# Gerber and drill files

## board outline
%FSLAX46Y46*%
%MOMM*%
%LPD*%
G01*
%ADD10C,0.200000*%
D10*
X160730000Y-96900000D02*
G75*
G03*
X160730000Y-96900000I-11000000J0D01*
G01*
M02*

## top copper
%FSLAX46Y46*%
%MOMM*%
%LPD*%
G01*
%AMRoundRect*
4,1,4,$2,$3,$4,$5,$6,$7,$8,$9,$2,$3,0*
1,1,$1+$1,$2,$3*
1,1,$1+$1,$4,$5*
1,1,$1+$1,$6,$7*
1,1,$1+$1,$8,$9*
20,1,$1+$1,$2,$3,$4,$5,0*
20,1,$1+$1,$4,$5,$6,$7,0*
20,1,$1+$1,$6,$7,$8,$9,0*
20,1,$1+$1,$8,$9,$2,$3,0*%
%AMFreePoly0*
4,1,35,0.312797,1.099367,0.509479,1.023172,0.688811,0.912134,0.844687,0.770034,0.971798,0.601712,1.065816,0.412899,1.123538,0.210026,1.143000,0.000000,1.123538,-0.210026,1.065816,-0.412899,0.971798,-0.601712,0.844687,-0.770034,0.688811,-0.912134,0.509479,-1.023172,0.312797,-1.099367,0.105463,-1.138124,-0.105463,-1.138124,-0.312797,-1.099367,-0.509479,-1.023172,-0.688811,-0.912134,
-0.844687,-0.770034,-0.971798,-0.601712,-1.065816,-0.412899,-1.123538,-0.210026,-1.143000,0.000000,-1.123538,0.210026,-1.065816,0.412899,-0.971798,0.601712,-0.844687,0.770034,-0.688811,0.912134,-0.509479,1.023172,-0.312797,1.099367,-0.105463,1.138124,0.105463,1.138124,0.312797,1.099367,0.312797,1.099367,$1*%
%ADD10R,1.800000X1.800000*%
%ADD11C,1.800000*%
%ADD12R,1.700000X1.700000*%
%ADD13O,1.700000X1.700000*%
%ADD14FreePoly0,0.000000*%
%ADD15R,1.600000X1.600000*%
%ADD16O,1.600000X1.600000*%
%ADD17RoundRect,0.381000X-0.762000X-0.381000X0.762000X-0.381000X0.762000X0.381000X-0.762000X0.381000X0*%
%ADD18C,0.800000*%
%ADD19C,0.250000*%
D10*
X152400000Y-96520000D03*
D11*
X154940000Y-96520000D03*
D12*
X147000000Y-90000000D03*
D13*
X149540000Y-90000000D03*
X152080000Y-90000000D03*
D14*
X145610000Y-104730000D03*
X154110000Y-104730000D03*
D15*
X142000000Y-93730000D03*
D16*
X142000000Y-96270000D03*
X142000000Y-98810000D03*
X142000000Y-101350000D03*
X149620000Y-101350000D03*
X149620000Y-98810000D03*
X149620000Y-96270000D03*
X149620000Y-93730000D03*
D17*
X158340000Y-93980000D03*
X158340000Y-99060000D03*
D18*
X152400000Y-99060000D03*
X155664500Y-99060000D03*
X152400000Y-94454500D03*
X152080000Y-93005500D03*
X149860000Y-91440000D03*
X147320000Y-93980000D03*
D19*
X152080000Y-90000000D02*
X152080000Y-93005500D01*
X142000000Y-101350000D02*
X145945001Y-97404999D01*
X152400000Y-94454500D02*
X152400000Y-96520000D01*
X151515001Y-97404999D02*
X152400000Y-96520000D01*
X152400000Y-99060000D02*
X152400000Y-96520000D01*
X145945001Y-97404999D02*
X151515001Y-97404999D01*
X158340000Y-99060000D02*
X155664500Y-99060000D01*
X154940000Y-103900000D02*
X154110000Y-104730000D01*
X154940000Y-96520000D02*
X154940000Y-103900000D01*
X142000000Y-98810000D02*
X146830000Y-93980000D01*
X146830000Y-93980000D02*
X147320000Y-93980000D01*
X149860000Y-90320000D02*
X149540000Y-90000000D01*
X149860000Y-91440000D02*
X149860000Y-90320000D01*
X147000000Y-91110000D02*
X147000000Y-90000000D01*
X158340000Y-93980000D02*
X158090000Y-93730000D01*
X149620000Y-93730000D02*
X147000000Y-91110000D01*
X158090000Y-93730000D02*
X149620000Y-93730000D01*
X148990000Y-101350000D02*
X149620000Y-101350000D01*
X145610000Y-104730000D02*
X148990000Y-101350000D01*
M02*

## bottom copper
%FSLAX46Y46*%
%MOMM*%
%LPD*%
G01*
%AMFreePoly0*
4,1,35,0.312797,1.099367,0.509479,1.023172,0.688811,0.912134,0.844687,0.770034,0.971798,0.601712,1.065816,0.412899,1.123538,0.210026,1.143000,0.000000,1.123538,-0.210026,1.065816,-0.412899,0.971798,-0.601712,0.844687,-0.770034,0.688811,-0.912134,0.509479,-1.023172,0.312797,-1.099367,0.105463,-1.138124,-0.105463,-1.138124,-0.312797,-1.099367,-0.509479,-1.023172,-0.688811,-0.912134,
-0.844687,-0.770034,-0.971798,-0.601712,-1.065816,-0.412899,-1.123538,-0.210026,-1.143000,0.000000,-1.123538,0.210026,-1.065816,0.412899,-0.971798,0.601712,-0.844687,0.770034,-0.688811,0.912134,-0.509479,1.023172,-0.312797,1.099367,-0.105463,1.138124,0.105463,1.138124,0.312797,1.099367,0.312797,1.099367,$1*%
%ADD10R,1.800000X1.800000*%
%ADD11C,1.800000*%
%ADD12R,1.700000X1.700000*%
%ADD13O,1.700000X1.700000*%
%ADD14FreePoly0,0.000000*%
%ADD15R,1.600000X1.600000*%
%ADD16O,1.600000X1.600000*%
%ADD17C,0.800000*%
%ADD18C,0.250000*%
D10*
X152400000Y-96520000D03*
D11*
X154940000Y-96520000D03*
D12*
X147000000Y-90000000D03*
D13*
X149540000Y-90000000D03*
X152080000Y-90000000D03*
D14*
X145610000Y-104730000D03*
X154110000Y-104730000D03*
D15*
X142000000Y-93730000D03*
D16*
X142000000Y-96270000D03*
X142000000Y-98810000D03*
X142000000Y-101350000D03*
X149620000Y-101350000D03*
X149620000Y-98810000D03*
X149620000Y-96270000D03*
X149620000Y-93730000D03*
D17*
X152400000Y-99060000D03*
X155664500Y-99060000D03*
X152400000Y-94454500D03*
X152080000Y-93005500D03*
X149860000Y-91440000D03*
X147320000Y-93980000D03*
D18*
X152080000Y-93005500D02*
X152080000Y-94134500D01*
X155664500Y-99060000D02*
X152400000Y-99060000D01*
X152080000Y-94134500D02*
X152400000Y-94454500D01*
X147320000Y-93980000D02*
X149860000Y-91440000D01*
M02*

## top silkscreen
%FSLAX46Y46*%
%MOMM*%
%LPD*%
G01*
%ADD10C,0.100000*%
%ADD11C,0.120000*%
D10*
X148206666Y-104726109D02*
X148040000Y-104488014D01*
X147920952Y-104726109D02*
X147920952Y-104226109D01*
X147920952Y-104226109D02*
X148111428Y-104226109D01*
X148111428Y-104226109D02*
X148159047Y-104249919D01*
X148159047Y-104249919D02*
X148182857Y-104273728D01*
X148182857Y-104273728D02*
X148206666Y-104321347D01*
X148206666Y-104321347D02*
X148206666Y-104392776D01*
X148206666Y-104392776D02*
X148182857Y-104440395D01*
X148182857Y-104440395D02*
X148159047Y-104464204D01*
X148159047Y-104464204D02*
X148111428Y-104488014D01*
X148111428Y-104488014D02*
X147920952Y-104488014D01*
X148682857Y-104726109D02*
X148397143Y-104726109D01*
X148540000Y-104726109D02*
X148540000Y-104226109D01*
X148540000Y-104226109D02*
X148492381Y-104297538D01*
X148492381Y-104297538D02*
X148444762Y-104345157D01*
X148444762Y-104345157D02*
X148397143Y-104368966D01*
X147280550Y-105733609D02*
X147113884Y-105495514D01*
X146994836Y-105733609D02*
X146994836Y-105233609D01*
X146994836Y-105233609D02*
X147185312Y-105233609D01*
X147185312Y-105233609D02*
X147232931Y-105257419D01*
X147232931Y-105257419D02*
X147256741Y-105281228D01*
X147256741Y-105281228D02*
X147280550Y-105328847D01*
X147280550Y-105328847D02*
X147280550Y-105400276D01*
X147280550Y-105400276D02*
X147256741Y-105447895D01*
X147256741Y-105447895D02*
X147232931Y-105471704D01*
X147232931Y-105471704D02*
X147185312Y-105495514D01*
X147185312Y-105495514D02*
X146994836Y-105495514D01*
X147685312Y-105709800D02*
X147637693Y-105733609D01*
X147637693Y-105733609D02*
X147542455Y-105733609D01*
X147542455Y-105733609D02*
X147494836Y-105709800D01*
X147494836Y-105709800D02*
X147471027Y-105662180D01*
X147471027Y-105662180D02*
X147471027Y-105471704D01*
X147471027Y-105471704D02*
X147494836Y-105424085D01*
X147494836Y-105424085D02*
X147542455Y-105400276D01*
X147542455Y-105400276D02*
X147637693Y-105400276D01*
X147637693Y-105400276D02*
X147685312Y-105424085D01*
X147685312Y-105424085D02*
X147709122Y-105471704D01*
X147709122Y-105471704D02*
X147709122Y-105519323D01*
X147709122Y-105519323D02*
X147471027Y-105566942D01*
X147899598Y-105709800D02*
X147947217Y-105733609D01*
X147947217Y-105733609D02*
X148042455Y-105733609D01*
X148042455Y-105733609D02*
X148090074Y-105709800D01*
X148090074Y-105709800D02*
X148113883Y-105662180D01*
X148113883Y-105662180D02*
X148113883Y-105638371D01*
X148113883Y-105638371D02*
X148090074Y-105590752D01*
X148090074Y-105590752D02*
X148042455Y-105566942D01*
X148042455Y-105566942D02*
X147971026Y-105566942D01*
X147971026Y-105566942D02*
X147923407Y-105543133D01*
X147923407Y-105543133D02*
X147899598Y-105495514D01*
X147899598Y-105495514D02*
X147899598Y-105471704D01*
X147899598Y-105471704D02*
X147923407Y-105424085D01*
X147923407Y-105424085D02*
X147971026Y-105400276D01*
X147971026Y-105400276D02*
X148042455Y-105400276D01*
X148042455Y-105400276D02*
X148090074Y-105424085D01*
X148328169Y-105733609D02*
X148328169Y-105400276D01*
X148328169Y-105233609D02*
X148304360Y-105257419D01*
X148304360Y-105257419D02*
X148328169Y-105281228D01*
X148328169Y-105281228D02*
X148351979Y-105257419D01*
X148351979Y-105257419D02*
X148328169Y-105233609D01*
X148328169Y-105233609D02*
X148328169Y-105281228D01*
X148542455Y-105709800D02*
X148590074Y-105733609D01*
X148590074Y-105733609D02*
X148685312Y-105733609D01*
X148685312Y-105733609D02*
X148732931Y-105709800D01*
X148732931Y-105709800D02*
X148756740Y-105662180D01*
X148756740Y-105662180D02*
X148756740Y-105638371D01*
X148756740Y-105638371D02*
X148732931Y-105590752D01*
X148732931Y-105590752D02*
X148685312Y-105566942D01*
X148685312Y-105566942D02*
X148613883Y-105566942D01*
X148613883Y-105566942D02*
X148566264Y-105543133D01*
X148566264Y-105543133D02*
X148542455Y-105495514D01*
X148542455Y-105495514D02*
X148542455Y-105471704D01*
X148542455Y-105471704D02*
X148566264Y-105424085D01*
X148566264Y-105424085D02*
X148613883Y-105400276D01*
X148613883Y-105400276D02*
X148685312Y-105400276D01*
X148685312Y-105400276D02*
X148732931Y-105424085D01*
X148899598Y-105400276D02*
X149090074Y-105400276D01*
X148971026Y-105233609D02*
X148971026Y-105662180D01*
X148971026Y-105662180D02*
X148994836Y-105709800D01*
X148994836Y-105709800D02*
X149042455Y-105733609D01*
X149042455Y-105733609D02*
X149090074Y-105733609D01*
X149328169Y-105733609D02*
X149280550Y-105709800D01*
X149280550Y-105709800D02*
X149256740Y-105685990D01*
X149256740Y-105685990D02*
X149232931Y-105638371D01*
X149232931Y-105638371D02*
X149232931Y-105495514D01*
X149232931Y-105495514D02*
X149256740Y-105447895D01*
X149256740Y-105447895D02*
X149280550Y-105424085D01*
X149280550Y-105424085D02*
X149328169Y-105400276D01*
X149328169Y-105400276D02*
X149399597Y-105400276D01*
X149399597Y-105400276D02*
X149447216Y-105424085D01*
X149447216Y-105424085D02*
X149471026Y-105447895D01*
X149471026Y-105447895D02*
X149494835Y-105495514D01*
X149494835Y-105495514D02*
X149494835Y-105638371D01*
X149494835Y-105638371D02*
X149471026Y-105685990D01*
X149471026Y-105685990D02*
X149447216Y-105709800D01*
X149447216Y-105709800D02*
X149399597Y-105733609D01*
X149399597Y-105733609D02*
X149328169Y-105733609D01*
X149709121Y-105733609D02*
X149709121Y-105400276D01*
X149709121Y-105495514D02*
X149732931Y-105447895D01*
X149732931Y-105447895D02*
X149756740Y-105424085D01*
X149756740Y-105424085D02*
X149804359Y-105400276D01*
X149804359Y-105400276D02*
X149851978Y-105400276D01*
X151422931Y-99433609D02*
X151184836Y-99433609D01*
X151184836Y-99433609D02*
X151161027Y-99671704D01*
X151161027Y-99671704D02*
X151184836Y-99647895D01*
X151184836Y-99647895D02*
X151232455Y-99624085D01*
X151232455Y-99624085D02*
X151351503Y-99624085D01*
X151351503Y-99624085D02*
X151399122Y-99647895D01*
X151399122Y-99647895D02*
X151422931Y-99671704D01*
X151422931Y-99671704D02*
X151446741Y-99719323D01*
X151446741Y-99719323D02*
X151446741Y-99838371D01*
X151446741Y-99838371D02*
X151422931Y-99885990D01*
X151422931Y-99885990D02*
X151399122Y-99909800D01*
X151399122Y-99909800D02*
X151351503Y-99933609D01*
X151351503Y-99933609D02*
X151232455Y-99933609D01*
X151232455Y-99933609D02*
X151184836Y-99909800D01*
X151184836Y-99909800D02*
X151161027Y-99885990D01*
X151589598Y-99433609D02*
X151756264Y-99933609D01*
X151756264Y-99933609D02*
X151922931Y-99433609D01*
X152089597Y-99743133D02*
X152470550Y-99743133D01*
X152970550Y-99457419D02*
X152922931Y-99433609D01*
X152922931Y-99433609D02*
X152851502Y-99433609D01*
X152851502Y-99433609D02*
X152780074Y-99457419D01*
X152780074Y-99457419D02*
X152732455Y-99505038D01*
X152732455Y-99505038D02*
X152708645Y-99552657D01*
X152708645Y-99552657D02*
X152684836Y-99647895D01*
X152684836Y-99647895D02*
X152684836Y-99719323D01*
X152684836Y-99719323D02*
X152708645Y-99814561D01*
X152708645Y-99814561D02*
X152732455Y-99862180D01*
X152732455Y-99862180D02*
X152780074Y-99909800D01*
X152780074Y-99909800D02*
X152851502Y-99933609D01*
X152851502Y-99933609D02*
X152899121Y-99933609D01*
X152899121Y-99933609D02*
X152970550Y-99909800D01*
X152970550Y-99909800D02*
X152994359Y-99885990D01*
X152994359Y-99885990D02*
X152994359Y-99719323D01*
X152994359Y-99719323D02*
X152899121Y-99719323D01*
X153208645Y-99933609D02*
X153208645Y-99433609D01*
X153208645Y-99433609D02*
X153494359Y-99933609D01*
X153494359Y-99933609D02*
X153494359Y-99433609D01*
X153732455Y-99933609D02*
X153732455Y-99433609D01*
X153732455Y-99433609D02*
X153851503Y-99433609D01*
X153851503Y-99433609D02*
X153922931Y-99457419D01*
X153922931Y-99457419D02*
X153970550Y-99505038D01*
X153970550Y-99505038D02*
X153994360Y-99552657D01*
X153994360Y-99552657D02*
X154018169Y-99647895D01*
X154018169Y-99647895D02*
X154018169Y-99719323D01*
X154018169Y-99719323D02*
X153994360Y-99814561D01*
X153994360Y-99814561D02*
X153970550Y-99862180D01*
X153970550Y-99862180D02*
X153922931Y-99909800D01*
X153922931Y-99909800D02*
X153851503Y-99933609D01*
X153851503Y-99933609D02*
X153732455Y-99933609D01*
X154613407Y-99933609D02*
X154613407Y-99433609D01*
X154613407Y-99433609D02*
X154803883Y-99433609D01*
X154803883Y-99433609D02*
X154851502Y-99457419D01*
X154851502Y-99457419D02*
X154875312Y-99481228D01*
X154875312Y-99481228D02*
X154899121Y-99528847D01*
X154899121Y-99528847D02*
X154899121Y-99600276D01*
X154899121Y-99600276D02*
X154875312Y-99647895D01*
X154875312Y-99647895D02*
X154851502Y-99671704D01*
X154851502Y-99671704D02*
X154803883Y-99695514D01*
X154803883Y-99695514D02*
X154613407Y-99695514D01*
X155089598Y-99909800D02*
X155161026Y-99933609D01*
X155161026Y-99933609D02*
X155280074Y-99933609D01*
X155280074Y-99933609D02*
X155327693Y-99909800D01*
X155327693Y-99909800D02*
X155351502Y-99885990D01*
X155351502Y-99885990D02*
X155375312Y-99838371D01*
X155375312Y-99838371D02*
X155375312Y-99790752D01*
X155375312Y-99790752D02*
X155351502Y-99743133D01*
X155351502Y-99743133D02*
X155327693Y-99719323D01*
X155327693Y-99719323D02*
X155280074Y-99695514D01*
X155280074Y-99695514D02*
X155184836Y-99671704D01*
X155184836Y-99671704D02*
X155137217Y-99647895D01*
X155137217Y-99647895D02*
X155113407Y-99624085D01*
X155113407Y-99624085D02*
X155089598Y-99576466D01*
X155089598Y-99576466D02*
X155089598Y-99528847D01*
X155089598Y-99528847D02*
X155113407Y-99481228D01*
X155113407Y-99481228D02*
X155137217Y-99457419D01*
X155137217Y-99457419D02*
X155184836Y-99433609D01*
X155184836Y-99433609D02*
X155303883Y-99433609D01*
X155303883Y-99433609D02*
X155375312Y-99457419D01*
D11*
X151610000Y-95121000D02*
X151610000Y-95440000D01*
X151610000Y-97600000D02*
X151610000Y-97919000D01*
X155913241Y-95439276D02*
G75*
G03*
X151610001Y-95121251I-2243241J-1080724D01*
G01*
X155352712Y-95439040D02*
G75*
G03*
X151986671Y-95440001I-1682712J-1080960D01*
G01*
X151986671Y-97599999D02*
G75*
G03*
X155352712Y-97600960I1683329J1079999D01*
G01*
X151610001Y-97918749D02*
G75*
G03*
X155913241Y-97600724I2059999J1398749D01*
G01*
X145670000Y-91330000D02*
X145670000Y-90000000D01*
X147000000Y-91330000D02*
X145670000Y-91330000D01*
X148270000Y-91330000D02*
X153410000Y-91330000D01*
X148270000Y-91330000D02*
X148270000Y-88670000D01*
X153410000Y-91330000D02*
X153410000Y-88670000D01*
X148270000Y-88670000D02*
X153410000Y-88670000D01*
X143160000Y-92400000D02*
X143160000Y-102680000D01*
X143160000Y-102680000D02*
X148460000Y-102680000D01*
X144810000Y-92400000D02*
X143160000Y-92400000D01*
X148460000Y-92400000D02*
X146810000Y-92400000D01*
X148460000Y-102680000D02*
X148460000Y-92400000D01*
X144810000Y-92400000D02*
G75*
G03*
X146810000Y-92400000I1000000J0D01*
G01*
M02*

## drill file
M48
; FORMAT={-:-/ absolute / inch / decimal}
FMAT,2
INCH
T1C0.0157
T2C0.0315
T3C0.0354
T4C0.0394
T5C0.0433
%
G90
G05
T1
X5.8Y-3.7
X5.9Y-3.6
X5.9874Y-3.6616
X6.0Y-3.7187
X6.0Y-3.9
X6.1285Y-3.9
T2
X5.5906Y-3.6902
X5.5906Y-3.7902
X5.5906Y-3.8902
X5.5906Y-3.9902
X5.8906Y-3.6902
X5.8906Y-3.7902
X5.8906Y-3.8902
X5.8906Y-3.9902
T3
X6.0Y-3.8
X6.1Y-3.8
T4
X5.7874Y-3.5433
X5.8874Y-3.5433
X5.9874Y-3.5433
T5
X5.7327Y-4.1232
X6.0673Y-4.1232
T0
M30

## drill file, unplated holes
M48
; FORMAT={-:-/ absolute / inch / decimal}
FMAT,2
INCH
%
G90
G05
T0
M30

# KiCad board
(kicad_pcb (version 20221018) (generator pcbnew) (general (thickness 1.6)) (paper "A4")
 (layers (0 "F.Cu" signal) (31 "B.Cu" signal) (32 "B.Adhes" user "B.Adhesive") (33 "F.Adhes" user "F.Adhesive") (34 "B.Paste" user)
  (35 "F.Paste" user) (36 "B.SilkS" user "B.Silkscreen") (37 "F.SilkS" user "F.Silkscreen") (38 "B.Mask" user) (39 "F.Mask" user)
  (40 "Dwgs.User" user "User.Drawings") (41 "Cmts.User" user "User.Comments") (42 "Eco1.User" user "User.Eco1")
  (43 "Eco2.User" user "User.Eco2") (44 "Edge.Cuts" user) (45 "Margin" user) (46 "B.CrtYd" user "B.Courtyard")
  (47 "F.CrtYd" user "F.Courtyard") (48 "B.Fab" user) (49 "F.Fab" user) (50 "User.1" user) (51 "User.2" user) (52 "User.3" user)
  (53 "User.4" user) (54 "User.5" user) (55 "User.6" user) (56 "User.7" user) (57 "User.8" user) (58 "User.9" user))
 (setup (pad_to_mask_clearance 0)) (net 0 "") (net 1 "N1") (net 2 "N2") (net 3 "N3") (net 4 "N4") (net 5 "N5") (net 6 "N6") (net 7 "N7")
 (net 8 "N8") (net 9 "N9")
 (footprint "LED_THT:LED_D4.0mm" (layer "F.Cu") (at 152.4 96.52)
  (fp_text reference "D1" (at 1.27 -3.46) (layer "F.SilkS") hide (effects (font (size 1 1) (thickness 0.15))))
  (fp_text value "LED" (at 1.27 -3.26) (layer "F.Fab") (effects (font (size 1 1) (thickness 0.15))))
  (fp_line (start -0.79 -1.399) (end -0.79 -1.08) (stroke (width 0.12) (type solid)) (layer "F.SilkS"))
  (fp_line (start -0.79 1.08) (end -0.79 1.399) (stroke (width 0.12) (type solid)) (layer "F.SilkS"))
  (fp_arc (start -0.79 -1.398749) (mid 1.453519 -2.483228) (end 3.513242 -1.080724) (stroke (width 0.12) (type solid)) (layer "F.SilkS"))
  (fp_arc (start -0.41333 -1.08) (mid 1.269429 -2) (end 2.952713 -1.080961) (stroke (width 0.12) (type solid)) (layer "F.SilkS"))
  (fp_arc (start 2.952713 1.080961) (mid 1.269429 2) (end -0.41333 1.08) (stroke (width 0.12) (type solid)) (layer "F.SilkS"))
  (fp_arc (start 3.513242 1.080724) (mid 1.453519 2.483228) (end -0.79 1.398749) (stroke (width 0.12) (type solid)) (layer "F.SilkS"))
  (pad "1" thru_hole rect (at 0 0) (size 1.8 1.8) (drill 0.9) (layers "*.Cu" "*.Mask") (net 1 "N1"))
  (pad "2" thru_hole circle (at 2.54 0) (size 1.8 1.8) (drill 0.9) (layers "*.Cu" "*.Mask") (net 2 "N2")))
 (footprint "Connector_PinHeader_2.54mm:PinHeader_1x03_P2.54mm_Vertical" (layer "F.Cu") (at 147 90 90)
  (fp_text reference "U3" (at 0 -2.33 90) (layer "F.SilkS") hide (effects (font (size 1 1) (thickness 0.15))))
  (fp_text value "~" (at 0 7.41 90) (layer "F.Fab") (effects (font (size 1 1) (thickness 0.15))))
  (fp_line (start -1.33 -1.33) (end 0 -1.33) (stroke (width 0.12) (type solid)) (layer "F.SilkS"))
  (fp_line (start -1.33 0) (end -1.33 -1.33) (stroke (width 0.12) (type solid)) (layer "F.SilkS"))
  (fp_line (start -1.33 1.27) (end -1.33 6.41) (stroke (width 0.12) (type solid)) (layer "F.SilkS"))
  (fp_line (start -1.33 1.27) (end 1.33 1.27) (stroke (width 0.12) (type solid)) (layer "F.SilkS"))
  (fp_line (start -1.33 6.41) (end 1.33 6.41) (stroke (width 0.12) (type solid)) (layer "F.SilkS"))
  (fp_line (start 1.33 1.27) (end 1.33 6.41) (stroke (width 0.12) (type solid)) (layer "F.SilkS"))
  (pad "1" thru_hole rect (at 0 0 90) (size 1.7 1.7) (drill 1) (layers "*.Cu" "*.Mask") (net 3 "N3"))
  (pad "2" thru_hole oval (at 0 2.54 90) (size 1.7 1.7) (drill 1) (layers "*.Cu" "*.Mask") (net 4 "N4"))
  (pad "3" thru_hole oval (at 0 5.08 90) (size 1.7 1.7) (drill 1) (layers "*.Cu" "*.Mask") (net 1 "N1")))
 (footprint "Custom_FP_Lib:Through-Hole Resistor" (layer "F.Cu") (at 145.29 106)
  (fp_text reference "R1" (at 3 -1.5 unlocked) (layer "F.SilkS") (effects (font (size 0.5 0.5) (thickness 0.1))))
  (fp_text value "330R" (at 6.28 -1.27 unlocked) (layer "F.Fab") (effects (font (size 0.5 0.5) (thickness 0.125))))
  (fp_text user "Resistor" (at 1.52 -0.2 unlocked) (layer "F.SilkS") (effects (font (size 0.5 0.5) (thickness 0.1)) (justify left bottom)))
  (pad "1" thru_hole custom (at 0.32 -1.27) (size 2.286 2.286) (drill 1.1) (layers "*.Cu" "*.Mask") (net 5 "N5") (thermal_bridge_angle 45)
   (options (clearance outline) (anchor circle)) (primitives))
  (pad "2" thru_hole custom (at 8.82 -1.27) (size 2.286 2.286) (drill 1.1) (layers "*.Cu" "*.Mask") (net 2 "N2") (thermal_bridge_angle 45)
   (options (clearance outline) (anchor circle)) (primitives)))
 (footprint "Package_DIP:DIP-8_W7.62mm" (layer "F.Cu") (at 142 93.73)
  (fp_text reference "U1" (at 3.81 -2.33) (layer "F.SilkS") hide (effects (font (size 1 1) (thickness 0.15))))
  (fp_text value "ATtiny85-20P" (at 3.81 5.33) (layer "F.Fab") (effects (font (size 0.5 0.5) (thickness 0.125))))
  (fp_line (start 1.16 -1.33) (end 1.16 8.95) (stroke (width 0.12) (type solid)) (layer "F.SilkS"))
  (fp_line (start 1.16 8.95) (end 6.46 8.95) (stroke (width 0.12) (type solid)) (layer "F.SilkS"))
  (fp_line (start 2.81 -1.33) (end 1.16 -1.33) (stroke (width 0.12) (type solid)) (layer "F.SilkS"))
  (fp_line (start 6.46 -1.33) (end 4.81 -1.33) (stroke (width 0.12) (type solid)) (layer "F.SilkS"))
  (fp_line (start 6.46 8.95) (end 6.46 -1.33) (stroke (width 0.12) (type solid)) (layer "F.SilkS"))
  (fp_arc (start 4.81 -1.33) (mid 3.81 -0.33) (end 2.81 -1.33) (stroke (width 0.12) (type solid)) (layer "F.SilkS"))
  (pad "1" thru_hole rect (at 0 0) (size 1.6 1.6) (drill 0.8) (layers "*.Cu" "*.Mask") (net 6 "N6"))
  (pad "2" thru_hole oval (at 0 2.54) (size 1.6 1.6) (drill 0.8) (layers "*.Cu" "*.Mask") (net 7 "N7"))
  (pad "3" thru_hole oval (at 0 5.08) (size 1.6 1.6) (drill 0.8) (layers "*.Cu" "*.Mask") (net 4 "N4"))
  (pad "4" thru_hole oval (at 0 7.62) (size 1.6 1.6) (drill 0.8) (layers "*.Cu" "*.Mask") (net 1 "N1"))
  (pad "5" thru_hole oval (at 7.62 7.62) (size 1.6 1.6) (drill 0.8) (layers "*.Cu" "*.Mask") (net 5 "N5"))
  (pad "6" thru_hole oval (at 7.62 5.08) (size 1.6 1.6) (drill 0.8) (layers "*.Cu" "*.Mask") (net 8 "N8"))
  (pad "7" thru_hole oval (at 7.62 2.54) (size 1.6 1.6) (drill 0.8) (layers "*.Cu" "*.Mask") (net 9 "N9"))
  (pad "8" thru_hole oval (at 7.62 0) (size 1.6 1.6) (drill 0.8) (layers "*.Cu" "*.Mask") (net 3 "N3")))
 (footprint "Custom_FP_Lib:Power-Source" (layer "F.Cu") (at 155.8 96.52)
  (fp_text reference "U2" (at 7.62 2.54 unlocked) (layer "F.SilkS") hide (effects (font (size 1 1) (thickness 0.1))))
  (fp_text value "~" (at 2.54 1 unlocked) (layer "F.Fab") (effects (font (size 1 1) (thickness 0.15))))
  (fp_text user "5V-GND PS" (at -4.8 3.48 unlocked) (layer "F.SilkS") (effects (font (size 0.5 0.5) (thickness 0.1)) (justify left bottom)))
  (pad "1" smd roundrect (at 2.54 -2.54) (size 2.286 1.524) (layers "F.Cu" "F.Paste" "F.Mask") (roundrect_rratio 0.25) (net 3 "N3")
   (thermal_bridge_angle 45))
  (pad "2" smd roundrect (at 2.54 2.54) (size 2.286 1.524) (layers "F.Cu" "F.Paste" "F.Mask") (roundrect_rratio 0.25) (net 1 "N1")
   (thermal_bridge_angle 45)))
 (gr_circle (center 149.73 96.9) (end 160.73 96.9) (stroke (width 0.2) (type default)) (fill none) (layer "Edge.Cuts"))
 (segment (start 152.08 90) (end 152.08 93.0055) (width 0.25) (layer "F.Cu") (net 1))
 (segment (start 142 101.35) (end 145.945001 97.404999) (width 0.25) (layer "F.Cu") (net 1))
 (segment (start 152.4 94.4545) (end 152.4 96.52) (width 0.25) (layer "F.Cu") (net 1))
 (segment (start 151.515001 97.404999) (end 152.4 96.52) (width 0.25) (layer "F.Cu") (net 1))
 (segment (start 152.4 99.06) (end 152.4 96.52) (width 0.25) (layer "F.Cu") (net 1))
 (segment (start 145.945001 97.404999) (end 151.515001 97.404999) (width 0.25) (layer "F.Cu") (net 1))
 (segment (start 158.34 99.06) (end 155.6645 99.06) (width 0.25) (layer "F.Cu") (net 1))
 (via (at 152.4 99.06) (size 0.8) (drill 0.4) (layers "F.Cu" "B.Cu") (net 1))
 (via (at 155.6645 99.06) (size 0.8) (drill 0.4) (layers "F.Cu" "B.Cu") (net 1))
 (via (at 152.4 94.4545) (size 0.8) (drill 0.4) (layers "F.Cu" "B.Cu") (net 1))
 (via (at 152.08 93.0055) (size 0.8) (drill 0.4) (layers "F.Cu" "B.Cu") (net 1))
 (segment (start 152.08 93.0055) (end 152.08 94.1345) (width 0.25) (layer "B.Cu") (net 1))
 (segment (start 155.6645 99.06) (end 152.4 99.06) (width 0.25) (layer "B.Cu") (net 1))
 (segment (start 152.08 94.1345) (end 152.4 94.4545) (width 0.25) (layer "B.Cu") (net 1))
 (segment (start 154.94 103.9) (end 154.11 104.73) (width 0.25) (layer "F.Cu") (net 2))
 (segment (start 154.94 96.52) (end 154.94 103.9) (width 0.25) (layer "F.Cu") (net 2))
 (segment (start 142 98.81) (end 146.83 93.98) (width 0.25) (layer "F.Cu") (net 4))
 (segment (start 146.83 93.98) (end 147.32 93.98) (width 0.25) (layer "F.Cu") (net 4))
 (segment (start 149.86 90.32) (end 149.54 90) (width 0.25) (layer "F.Cu") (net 4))
 (segment (start 149.86 91.44) (end 149.86 90.32) (width 0.25) (layer "F.Cu") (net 4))
 (via (at 149.86 91.44) (size 0.8) (drill 0.4) (layers "F.Cu" "B.Cu") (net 4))
 (via (at 147.32 93.98) (size 0.8) (drill 0.4) (layers "F.Cu" "B.Cu") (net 4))
 (segment (start 147.32 93.98) (end 149.86 91.44) (width 0.25) (layer "B.Cu") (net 4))
 (segment (start 147 91.11) (end 147 90) (width 0.25) (layer "F.Cu") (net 3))
 (segment (start 158.34 93.98) (end 158.09 93.73) (width 0.25) (layer "F.Cu") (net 3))
 (segment (start 149.62 93.73) (end 147 91.11) (width 0.25) (layer "F.Cu") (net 3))
 (segment (start 158.09 93.73) (end 149.62 93.73) (width 0.25) (layer "F.Cu") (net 3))
 (segment (start 148.99 101.35) (end 149.62 101.35) (width 0.25) (layer "F.Cu") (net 5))
 (segment (start 145.61 104.73) (end 148.99 101.35) (width 0.25) (layer "F.Cu") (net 5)))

